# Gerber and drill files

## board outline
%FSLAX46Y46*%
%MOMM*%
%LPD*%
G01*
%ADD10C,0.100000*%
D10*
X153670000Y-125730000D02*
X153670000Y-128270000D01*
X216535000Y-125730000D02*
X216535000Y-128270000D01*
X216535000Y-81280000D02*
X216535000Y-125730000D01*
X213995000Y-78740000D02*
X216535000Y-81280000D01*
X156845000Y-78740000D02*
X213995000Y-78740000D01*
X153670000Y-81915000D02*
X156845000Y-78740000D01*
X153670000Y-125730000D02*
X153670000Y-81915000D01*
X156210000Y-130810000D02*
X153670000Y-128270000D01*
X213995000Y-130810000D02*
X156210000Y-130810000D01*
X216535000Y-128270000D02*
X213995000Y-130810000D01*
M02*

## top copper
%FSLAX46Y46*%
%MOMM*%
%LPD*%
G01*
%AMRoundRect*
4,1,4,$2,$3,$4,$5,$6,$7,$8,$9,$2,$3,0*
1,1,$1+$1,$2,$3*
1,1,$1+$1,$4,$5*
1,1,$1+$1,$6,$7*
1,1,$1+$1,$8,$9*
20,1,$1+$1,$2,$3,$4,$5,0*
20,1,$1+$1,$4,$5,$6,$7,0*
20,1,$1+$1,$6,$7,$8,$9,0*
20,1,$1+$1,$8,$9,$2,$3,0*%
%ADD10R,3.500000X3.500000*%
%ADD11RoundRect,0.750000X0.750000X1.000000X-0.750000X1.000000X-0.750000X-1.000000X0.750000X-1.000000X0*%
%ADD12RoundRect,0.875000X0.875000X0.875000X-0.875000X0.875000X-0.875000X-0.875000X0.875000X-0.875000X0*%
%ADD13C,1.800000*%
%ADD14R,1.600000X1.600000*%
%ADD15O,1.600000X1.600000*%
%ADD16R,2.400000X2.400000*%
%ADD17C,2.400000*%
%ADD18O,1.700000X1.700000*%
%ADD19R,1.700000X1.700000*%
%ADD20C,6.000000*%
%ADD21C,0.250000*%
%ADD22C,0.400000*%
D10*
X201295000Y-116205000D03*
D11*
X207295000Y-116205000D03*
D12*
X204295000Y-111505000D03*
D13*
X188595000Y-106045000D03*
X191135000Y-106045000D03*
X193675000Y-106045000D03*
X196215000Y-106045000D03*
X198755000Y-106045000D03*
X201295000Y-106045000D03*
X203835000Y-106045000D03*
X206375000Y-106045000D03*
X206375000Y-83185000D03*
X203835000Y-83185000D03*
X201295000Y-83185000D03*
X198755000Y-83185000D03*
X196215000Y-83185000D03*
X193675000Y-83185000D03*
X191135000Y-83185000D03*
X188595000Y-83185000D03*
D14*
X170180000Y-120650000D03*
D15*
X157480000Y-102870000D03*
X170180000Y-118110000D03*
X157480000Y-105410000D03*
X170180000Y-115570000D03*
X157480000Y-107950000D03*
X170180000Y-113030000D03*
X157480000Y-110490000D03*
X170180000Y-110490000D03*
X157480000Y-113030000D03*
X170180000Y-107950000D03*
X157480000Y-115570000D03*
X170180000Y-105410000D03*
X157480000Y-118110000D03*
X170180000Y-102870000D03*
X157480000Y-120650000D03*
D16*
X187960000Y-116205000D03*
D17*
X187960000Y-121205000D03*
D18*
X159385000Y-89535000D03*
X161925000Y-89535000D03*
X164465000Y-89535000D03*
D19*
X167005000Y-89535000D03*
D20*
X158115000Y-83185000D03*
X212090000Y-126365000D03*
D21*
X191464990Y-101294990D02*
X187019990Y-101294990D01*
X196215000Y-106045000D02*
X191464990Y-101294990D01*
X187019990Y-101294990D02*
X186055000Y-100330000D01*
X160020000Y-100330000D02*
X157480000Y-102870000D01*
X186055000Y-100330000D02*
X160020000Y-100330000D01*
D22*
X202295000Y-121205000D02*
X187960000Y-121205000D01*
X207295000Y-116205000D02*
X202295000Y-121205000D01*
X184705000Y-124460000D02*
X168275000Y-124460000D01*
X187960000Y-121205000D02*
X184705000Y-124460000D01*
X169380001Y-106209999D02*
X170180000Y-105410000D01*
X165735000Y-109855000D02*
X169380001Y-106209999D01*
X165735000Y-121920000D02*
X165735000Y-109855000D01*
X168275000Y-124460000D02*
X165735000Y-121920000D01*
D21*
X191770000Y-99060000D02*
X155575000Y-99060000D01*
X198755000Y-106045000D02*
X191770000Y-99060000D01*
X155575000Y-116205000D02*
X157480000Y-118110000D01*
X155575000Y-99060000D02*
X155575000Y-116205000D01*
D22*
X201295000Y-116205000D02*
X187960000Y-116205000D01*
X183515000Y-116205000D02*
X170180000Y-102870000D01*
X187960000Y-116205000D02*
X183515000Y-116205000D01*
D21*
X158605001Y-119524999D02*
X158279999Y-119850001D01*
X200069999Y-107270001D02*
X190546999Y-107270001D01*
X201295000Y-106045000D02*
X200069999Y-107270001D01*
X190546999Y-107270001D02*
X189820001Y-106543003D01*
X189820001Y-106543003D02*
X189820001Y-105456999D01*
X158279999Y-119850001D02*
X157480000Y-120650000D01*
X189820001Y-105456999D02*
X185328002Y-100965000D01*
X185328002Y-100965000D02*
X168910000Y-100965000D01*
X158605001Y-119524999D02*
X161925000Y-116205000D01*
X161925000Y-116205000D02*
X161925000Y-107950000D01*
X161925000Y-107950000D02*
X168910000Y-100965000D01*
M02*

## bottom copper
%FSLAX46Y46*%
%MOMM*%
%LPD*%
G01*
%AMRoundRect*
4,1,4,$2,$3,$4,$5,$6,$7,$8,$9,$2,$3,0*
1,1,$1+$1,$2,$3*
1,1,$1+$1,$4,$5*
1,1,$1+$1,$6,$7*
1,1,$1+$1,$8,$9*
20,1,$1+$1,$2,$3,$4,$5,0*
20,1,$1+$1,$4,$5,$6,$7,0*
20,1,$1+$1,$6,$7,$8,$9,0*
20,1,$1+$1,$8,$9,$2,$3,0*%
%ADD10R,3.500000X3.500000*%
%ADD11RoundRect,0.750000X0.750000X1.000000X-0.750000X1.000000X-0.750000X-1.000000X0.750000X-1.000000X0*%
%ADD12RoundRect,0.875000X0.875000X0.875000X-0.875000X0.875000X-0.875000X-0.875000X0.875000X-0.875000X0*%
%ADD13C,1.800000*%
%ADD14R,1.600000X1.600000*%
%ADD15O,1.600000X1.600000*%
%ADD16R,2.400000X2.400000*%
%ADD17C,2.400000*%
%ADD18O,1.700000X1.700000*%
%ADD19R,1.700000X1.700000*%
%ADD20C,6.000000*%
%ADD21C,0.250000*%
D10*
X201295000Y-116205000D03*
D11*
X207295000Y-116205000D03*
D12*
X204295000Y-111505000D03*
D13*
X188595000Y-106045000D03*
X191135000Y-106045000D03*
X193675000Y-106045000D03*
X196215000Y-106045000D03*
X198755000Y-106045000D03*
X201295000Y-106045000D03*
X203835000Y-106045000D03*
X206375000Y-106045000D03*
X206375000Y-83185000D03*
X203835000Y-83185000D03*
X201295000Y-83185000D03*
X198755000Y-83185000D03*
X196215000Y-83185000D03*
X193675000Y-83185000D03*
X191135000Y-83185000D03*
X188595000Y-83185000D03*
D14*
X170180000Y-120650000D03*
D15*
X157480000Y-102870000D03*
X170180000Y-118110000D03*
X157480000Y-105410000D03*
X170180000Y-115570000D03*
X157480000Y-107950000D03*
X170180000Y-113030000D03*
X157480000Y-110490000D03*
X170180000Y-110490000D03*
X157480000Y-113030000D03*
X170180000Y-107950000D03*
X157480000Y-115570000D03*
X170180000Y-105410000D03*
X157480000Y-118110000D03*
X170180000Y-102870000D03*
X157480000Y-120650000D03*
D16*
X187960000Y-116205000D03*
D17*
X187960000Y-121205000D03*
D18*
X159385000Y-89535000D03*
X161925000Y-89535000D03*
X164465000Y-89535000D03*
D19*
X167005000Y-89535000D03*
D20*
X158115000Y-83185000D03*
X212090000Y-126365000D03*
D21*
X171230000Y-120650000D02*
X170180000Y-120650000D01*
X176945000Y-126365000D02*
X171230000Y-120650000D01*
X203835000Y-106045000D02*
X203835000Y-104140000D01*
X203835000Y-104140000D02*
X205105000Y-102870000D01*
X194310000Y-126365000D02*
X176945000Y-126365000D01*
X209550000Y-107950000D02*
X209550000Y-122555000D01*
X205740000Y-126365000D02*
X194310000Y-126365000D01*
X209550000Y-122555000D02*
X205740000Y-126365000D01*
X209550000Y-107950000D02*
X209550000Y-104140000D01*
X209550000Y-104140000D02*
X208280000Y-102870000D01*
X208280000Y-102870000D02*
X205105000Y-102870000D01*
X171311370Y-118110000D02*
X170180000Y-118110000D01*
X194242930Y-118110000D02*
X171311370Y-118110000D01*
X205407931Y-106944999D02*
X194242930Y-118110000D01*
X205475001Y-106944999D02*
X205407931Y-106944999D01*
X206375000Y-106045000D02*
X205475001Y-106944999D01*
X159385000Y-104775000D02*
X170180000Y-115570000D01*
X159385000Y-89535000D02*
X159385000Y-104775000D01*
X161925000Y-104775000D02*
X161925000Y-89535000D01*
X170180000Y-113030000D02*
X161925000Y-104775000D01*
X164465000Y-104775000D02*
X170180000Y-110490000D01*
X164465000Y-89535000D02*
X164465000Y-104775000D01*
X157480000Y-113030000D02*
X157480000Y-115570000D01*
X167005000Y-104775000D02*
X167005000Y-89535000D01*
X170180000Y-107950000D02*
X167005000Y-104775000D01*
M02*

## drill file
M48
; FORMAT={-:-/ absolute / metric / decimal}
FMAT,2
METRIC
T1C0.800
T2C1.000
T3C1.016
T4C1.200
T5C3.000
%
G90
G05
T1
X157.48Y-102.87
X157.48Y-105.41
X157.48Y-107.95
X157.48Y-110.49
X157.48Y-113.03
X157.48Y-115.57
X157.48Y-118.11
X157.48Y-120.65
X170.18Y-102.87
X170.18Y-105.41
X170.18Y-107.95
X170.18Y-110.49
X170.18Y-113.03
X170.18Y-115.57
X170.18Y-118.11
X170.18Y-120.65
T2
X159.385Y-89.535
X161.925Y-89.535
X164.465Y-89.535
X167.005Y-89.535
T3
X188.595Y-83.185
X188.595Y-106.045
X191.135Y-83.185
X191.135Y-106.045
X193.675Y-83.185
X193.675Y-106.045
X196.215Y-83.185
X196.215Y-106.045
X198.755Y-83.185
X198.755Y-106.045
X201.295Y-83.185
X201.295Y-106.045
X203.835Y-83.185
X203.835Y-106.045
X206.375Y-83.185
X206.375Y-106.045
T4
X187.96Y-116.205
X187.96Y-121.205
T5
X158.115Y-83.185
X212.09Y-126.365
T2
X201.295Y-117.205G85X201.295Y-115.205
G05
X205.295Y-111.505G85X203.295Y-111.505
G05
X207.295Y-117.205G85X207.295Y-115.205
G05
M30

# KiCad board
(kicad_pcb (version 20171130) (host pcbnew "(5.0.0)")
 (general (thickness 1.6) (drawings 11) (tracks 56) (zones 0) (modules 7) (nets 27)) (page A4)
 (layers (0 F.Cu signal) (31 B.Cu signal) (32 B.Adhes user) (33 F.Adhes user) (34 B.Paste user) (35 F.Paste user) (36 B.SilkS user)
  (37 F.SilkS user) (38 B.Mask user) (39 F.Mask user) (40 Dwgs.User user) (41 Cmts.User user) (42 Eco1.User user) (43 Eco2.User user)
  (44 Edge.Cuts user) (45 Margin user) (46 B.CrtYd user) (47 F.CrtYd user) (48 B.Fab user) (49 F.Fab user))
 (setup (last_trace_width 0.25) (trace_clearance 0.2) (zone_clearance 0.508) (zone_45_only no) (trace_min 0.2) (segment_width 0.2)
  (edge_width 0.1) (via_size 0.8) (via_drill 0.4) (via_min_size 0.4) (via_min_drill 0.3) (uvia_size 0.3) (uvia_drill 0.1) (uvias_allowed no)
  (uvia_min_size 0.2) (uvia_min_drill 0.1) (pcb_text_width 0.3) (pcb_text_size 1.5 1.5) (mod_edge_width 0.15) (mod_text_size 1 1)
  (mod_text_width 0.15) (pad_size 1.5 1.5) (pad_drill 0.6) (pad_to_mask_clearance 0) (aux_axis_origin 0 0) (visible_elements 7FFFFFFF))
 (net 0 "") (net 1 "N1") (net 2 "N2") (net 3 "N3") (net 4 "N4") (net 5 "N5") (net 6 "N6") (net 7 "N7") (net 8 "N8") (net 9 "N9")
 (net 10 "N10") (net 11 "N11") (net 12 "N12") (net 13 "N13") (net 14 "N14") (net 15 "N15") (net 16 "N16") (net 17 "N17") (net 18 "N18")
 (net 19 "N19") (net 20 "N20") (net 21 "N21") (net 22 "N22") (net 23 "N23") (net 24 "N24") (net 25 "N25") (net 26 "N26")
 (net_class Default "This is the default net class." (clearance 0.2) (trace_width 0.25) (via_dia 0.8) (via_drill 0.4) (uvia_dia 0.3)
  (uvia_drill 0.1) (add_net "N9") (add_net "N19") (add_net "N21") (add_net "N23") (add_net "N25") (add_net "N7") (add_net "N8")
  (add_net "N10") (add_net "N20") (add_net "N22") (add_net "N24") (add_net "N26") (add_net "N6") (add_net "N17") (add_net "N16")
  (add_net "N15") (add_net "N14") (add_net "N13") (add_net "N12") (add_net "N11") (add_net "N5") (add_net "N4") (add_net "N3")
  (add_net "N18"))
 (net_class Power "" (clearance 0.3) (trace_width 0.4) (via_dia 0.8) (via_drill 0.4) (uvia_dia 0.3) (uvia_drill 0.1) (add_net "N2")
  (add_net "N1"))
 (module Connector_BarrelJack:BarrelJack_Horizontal (layer F.Cu) (at 201.295 116.205 180)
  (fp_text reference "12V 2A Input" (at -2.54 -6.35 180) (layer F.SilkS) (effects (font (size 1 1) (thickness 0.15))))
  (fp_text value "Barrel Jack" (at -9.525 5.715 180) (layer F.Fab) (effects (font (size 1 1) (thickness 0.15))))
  (pad 1 thru_hole rect (at 0 0 180) (size 3.5 3.5) (drill oval 1 3) (layers *.Cu *.Mask) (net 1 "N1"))
  (pad 2 thru_hole roundrect (at -6 0 180) (size 3 3.5) (drill oval 1 3) (layers *.Cu *.Mask) (roundrect_rratio 0.25) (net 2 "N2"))
  (pad 3 thru_hole roundrect (at -3 4.7 180) (size 3.5 3.5) (drill oval 3 1) (layers *.Cu *.Mask) (roundrect_rratio 0.25)))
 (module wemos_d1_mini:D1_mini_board (layer F.Cu) (at 198.755 94.615 90)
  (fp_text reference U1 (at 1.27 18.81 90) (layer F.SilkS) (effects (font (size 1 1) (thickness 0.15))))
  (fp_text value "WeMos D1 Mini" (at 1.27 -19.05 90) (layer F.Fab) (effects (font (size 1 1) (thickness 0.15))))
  (pad 8 thru_hole circle (at -11.43 -10.16 90) (size 1.8 1.8) (drill 1.016) (layers *.Cu *.Mask F.SilkS) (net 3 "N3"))
  (pad 7 thru_hole circle (at -11.43 -7.62 90) (size 1.8 1.8) (drill 1.016) (layers *.Cu *.Mask F.SilkS) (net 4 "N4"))
  (pad 6 thru_hole circle (at -11.43 -5.08 90) (size 1.8 1.8) (drill 1.016) (layers *.Cu *.Mask F.SilkS) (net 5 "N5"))
  (pad 5 thru_hole circle (at -11.43 -2.54 90) (size 1.8 1.8) (drill 1.016) (layers *.Cu *.Mask F.SilkS) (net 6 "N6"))
  (pad 4 thru_hole circle (at -11.43 0 90) (size 1.8 1.8) (drill 1.016) (layers *.Cu *.Mask F.SilkS) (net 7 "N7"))
  (pad 3 thru_hole circle (at -11.43 2.54 90) (size 1.8 1.8) (drill 1.016) (layers *.Cu *.Mask F.SilkS) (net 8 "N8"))
  (pad 2 thru_hole circle (at -11.43 5.08 90) (size 1.8 1.8) (drill 1.016) (layers *.Cu *.Mask F.SilkS) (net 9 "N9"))
  (pad 1 thru_hole circle (at -11.43 7.62 90) (size 1.8 1.8) (drill 1.016) (layers *.Cu *.Mask F.SilkS) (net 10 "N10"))
  (pad 16 thru_hole circle (at 11.43 7.62 90) (size 1.8 1.8) (drill 1.016) (layers *.Cu *.Mask F.SilkS) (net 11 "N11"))
  (pad 15 thru_hole circle (at 11.43 5.08 90) (size 1.8 1.8) (drill 1.016) (layers *.Cu *.Mask F.SilkS) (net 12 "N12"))
  (pad 14 thru_hole circle (at 11.43 2.54 90) (size 1.8 1.8) (drill 1.016) (layers *.Cu *.Mask F.SilkS) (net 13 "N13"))
  (pad 13 thru_hole circle (at 11.43 0 90) (size 1.8 1.8) (drill 1.016) (layers *.Cu *.Mask F.SilkS) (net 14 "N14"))
  (pad 12 thru_hole circle (at 11.43 -2.54 90) (size 1.8 1.8) (drill 1.016) (layers *.Cu *.Mask F.SilkS) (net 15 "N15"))
  (pad 11 thru_hole circle (at 11.43 -5.08 90) (size 1.8 1.8) (drill 1.016) (layers *.Cu *.Mask F.SilkS) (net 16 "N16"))
  (pad 10 thru_hole circle (at 11.43 -7.62 90) (size 1.8 1.8) (drill 1.016) (layers *.Cu *.Mask F.SilkS) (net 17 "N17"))
  (pad 9 thru_hole circle (at 11.43 -10.16 90) (size 1.8 1.8) (drill 1.016) (layers *.Cu *.Mask F.SilkS) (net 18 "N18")))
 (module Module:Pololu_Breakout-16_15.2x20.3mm (layer F.Cu) (at 170.18 120.65 180)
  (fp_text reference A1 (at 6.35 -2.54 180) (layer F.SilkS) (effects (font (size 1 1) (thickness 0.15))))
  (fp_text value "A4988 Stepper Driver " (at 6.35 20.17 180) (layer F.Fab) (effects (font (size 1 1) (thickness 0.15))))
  (pad 1 thru_hole rect (at 0 0 180) (size 1.6 1.6) (drill 0.8) (layers *.Cu *.Mask) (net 9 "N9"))
  (pad 9 thru_hole oval (at 12.7 17.78 180) (size 1.6 1.6) (drill 0.8) (layers *.Cu *.Mask) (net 6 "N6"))
  (pad 2 thru_hole oval (at 0 2.54 180) (size 1.6 1.6) (drill 0.8) (layers *.Cu *.Mask) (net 10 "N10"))
  (pad 10 thru_hole oval (at 12.7 15.24 180) (size 1.6 1.6) (drill 0.8) (layers *.Cu *.Mask) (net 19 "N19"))
  (pad 3 thru_hole oval (at 0 5.08 180) (size 1.6 1.6) (drill 0.8) (layers *.Cu *.Mask) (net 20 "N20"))
  (pad 11 thru_hole oval (at 12.7 12.7 180) (size 1.6 1.6) (drill 0.8) (layers *.Cu *.Mask) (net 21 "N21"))
  (pad 4 thru_hole oval (at 0 7.62 180) (size 1.6 1.6) (drill 0.8) (layers *.Cu *.Mask) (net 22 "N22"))
  (pad 12 thru_hole oval (at 12.7 10.16 180) (size 1.6 1.6) (drill 0.8) (layers *.Cu *.Mask) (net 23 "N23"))
  (pad 5 thru_hole oval (at 0 10.16 180) (size 1.6 1.6) (drill 0.8) (layers *.Cu *.Mask) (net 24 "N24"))
  (pad 13 thru_hole oval (at 12.7 7.62 180) (size 1.6 1.6) (drill 0.8) (layers *.Cu *.Mask) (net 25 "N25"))
  (pad 6 thru_hole oval (at 0 12.7 180) (size 1.6 1.6) (drill 0.8) (layers *.Cu *.Mask) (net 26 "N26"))
  (pad 14 thru_hole oval (at 12.7 5.08 180) (size 1.6 1.6) (drill 0.8) (layers *.Cu *.Mask) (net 25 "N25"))
  (pad 7 thru_hole oval (at 0 15.24 180) (size 1.6 1.6) (drill 0.8) (layers *.Cu *.Mask) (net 2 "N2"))
  (pad 15 thru_hole oval (at 12.7 2.54 180) (size 1.6 1.6) (drill 0.8) (layers *.Cu *.Mask) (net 7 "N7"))
  (pad 8 thru_hole oval (at 0 17.78 180) (size 1.6 1.6) (drill 0.8) (layers *.Cu *.Mask) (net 1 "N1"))
  (pad 16 thru_hole oval (at 12.7 0 180) (size 1.6 1.6) (drill 0.8) (layers *.Cu *.Mask) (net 8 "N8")))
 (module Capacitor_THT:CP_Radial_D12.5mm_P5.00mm (layer F.Cu) (at 187.96 116.205 270)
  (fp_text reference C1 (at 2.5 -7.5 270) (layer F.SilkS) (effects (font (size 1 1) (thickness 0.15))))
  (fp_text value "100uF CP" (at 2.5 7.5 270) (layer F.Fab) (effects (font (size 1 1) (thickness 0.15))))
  (pad 1 thru_hole rect (at 0 0 270) (size 2.4 2.4) (drill 1.2) (layers *.Cu *.Mask) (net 1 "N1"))
  (pad 2 thru_hole circle (at 5 0 270) (size 2.4 2.4) (drill 1.2) (layers *.Cu *.Mask) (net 2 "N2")))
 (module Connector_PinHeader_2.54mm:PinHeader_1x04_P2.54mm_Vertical (layer F.Cu) (at 167.005 89.535 270)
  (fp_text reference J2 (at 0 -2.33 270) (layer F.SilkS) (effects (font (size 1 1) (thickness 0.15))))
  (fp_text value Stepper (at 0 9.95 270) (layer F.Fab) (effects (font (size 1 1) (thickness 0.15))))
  (pad 4 thru_hole oval (at 0 7.62 270) (size 1.7 1.7) (drill 1) (layers *.Cu *.Mask) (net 20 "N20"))
  (pad 3 thru_hole oval (at 0 5.08 270) (size 1.7 1.7) (drill 1) (layers *.Cu *.Mask) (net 22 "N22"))
  (pad 2 thru_hole oval (at 0 2.54 270) (size 1.7 1.7) (drill 1) (layers *.Cu *.Mask) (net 24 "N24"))
  (pad 1 thru_hole rect (at 0 0 270) (size 1.7 1.7) (drill 1) (layers *.Cu *.Mask) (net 26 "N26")))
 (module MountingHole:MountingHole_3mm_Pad (layer F.Cu) (at 158.115 83.185)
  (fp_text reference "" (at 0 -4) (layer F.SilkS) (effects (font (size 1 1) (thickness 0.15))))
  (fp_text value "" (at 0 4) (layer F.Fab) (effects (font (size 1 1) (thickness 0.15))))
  (pad 1 thru_hole circle (at 0 0) (size 6 6) (drill 3) (layers *.Cu *.Mask)))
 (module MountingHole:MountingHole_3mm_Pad (layer F.Cu) (at 212.09 126.365)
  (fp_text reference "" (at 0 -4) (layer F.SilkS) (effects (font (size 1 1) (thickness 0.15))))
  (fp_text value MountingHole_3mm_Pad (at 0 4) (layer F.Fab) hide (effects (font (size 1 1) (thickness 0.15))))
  (pad 1 thru_hole circle (at 0 0) (size 6 6) (drill 3) (layers *.Cu *.Mask)))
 (gr_line (start 153.67 125.73) (end 153.67 128.27) (layer Edge.Cuts) (width 0.1))
 (gr_line (start 216.535 125.73) (end 216.535 128.27) (layer Edge.Cuts) (width 0.1))
 (gr_line (start 216.535 81.28) (end 216.535 125.73) (layer Edge.Cuts) (width 0.1))
 (gr_line (start 213.995 78.74) (end 216.535 81.28) (layer Edge.Cuts) (width 0.1))
 (gr_line (start 156.845 78.74) (end 213.995 78.74) (layer Edge.Cuts) (width 0.1))
 (gr_line (start 153.67 81.915) (end 156.845 78.74) (layer Edge.Cuts) (width 0.1))
 (gr_line (start 153.67 125.73) (end 153.67 81.915) (layer Edge.Cuts) (width 0.1))
 (gr_line (start 156.21 130.81) (end 153.67 128.27) (layer Edge.Cuts) (width 0.1))
 (gr_line (start 213.995 130.81) (end 156.21 130.81) (layer Edge.Cuts) (width 0.1))
 (gr_line (start 216.535 128.27) (end 213.995 130.81) (layer Edge.Cuts) (width 0.1))
 (segment (start 171.23 120.65) (end 170.18 120.65) (width 0.25) (layer B.Cu) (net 9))
 (segment (start 176.945 126.365) (end 171.23 120.65) (width 0.25) (layer B.Cu) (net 9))
 (segment (start 203.835 106.045) (end 203.835 104.14) (width 0.25) (layer B.Cu) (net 9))
 (segment (start 203.835 104.14) (end 205.105 102.87) (width 0.25) (layer B.Cu) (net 9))
 (segment (start 194.31 126.365) (end 176.945 126.365) (width 0.25) (layer B.Cu) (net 9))
 (segment (start 209.55 107.95) (end 209.55 122.555) (width 0.25) (layer B.Cu) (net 9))
 (segment (start 205.74 126.365) (end 194.31 126.365) (width 0.25) (layer B.Cu) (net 9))
 (segment (start 209.55 122.555) (end 205.74 126.365) (width 0.25) (layer B.Cu) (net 9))
 (segment (start 209.55 107.95) (end 209.55 104.14) (width 0.25) (layer B.Cu) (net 9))
 (segment (start 209.55 104.14) (end 208.28 102.87) (width 0.25) (layer B.Cu) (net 9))
 (segment (start 208.28 102.87) (end 205.105 102.87) (width 0.25) (layer B.Cu) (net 9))
 (segment (start 191.46499 101.29499) (end 187.01999 101.29499) (width 0.25) (layer F.Cu) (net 6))
 (segment (start 196.215 106.045) (end 191.46499 101.29499) (width 0.25) (layer F.Cu) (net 6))
 (segment (start 187.01999 101.29499) (end 186.055 100.33) (width 0.25) (layer F.Cu) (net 6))
 (segment (start 160.02 100.33) (end 157.48 102.87) (width 0.25) (layer F.Cu) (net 6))
 (segment (start 186.055 100.33) (end 160.02 100.33) (width 0.25) (layer F.Cu) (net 6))
 (segment (start 171.31137 118.11) (end 170.18 118.11) (width 0.25) (layer B.Cu) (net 10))
 (segment (start 194.24293 118.11) (end 171.31137 118.11) (width 0.25) (layer B.Cu) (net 10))
 (segment (start 205.407931 106.944999) (end 194.24293 118.11) (width 0.25) (layer B.Cu) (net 10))
 (segment (start 205.475001 106.944999) (end 205.407931 106.944999) (width 0.25) (layer B.Cu) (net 10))
 (segment (start 206.375 106.045) (end 205.475001 106.944999) (width 0.25) (layer B.Cu) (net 10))
 (segment (start 159.385 104.775) (end 170.18 115.57) (width 0.25) (layer B.Cu) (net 20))
 (segment (start 159.385 89.535) (end 159.385 104.775) (width 0.25) (layer B.Cu) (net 20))
 (segment (start 161.925 104.775) (end 161.925 89.535) (width 0.25) (layer B.Cu) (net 22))
 (segment (start 170.18 113.03) (end 161.925 104.775) (width 0.25) (layer B.Cu) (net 22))
 (segment (start 164.465 104.775) (end 170.18 110.49) (width 0.25) (layer B.Cu) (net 24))
 (segment (start 164.465 89.535) (end 164.465 104.775) (width 0.25) (layer B.Cu) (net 24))
 (segment (start 157.48 113.03) (end 157.48 115.57) (width 0.25) (layer B.Cu) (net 25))
 (segment (start 167.005 104.775) (end 167.005 89.535) (width 0.25) (layer B.Cu) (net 26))
 (segment (start 170.18 107.95) (end 167.005 104.775) (width 0.25) (layer B.Cu) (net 26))
 (segment (start 202.295 121.205) (end 187.96 121.205) (width 0.4) (layer F.Cu) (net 2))
 (segment (start 207.295 116.205) (end 202.295 121.205) (width 0.4) (layer F.Cu) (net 2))
 (segment (start 184.705 124.46) (end 168.275 124.46) (width 0.4) (layer F.Cu) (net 2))
 (segment (start 187.96 121.205) (end 184.705 124.46) (width 0.4) (layer F.Cu) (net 2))
 (segment (start 169.380001 106.209999) (end 170.18 105.41) (width 0.4) (layer F.Cu) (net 2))
 (segment (start 165.735 109.855) (end 169.380001 106.209999) (width 0.4) (layer F.Cu) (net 2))
 (segment (start 165.735 121.92) (end 165.735 109.855) (width 0.4) (layer F.Cu) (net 2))
 (segment (start 168.275 124.46) (end 165.735 121.92) (width 0.4) (layer F.Cu) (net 2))
 (segment (start 191.77 99.06) (end 155.575 99.06) (width 0.25) (layer F.Cu) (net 7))
 (segment (start 198.755 106.045) (end 191.77 99.06) (width 0.25) (layer F.Cu) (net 7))
 (segment (start 155.575 116.205) (end 157.48 118.11) (width 0.25) (layer F.Cu) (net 7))
 (segment (start 155.575 99.06) (end 155.575 116.205) (width 0.25) (layer F.Cu) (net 7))
 (segment (start 201.295 116.205) (end 187.96 116.205) (width 0.4) (layer F.Cu) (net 1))
 (segment (start 183.515 116.205) (end 170.18 102.87) (width 0.4) (layer F.Cu) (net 1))
 (segment (start 187.96 116.205) (end 183.515 116.205) (width 0.4) (layer F.Cu) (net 1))
 (segment (start 158.605001 119.524999) (end 158.279999 119.850001) (width 0.25) (layer F.Cu) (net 8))
 (segment (start 200.069999 107.270001) (end 190.546999 107.270001) (width 0.25) (layer F.Cu) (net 8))
 (segment (start 201.295 106.045) (end 200.069999 107.270001) (width 0.25) (layer F.Cu) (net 8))
 (segment (start 190.546999 107.270001) (end 189.820001 106.543003) (width 0.25) (layer F.Cu) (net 8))
 (segment (start 189.820001 106.543003) (end 189.820001 105.456999) (width 0.25) (layer F.Cu) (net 8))
 (segment (start 158.279999 119.850001) (end 157.48 120.65) (width 0.25) (layer F.Cu) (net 8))
 (segment (start 189.820001 105.456999) (end 185.328002 100.965) (width 0.25) (layer F.Cu) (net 8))
 (segment (start 185.328002 100.965) (end 168.91 100.965) (width 0.25) (layer F.Cu) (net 8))
 (segment (start 158.605001 119.524999) (end 161.925 116.205) (width 0.25) (layer F.Cu) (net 8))
 (segment (start 161.925 116.205) (end 161.925 107.95) (width 0.25) (layer F.Cu) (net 8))
 (segment (start 161.925 107.95) (end 168.91 100.965) (width 0.25) (layer F.Cu) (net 8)))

